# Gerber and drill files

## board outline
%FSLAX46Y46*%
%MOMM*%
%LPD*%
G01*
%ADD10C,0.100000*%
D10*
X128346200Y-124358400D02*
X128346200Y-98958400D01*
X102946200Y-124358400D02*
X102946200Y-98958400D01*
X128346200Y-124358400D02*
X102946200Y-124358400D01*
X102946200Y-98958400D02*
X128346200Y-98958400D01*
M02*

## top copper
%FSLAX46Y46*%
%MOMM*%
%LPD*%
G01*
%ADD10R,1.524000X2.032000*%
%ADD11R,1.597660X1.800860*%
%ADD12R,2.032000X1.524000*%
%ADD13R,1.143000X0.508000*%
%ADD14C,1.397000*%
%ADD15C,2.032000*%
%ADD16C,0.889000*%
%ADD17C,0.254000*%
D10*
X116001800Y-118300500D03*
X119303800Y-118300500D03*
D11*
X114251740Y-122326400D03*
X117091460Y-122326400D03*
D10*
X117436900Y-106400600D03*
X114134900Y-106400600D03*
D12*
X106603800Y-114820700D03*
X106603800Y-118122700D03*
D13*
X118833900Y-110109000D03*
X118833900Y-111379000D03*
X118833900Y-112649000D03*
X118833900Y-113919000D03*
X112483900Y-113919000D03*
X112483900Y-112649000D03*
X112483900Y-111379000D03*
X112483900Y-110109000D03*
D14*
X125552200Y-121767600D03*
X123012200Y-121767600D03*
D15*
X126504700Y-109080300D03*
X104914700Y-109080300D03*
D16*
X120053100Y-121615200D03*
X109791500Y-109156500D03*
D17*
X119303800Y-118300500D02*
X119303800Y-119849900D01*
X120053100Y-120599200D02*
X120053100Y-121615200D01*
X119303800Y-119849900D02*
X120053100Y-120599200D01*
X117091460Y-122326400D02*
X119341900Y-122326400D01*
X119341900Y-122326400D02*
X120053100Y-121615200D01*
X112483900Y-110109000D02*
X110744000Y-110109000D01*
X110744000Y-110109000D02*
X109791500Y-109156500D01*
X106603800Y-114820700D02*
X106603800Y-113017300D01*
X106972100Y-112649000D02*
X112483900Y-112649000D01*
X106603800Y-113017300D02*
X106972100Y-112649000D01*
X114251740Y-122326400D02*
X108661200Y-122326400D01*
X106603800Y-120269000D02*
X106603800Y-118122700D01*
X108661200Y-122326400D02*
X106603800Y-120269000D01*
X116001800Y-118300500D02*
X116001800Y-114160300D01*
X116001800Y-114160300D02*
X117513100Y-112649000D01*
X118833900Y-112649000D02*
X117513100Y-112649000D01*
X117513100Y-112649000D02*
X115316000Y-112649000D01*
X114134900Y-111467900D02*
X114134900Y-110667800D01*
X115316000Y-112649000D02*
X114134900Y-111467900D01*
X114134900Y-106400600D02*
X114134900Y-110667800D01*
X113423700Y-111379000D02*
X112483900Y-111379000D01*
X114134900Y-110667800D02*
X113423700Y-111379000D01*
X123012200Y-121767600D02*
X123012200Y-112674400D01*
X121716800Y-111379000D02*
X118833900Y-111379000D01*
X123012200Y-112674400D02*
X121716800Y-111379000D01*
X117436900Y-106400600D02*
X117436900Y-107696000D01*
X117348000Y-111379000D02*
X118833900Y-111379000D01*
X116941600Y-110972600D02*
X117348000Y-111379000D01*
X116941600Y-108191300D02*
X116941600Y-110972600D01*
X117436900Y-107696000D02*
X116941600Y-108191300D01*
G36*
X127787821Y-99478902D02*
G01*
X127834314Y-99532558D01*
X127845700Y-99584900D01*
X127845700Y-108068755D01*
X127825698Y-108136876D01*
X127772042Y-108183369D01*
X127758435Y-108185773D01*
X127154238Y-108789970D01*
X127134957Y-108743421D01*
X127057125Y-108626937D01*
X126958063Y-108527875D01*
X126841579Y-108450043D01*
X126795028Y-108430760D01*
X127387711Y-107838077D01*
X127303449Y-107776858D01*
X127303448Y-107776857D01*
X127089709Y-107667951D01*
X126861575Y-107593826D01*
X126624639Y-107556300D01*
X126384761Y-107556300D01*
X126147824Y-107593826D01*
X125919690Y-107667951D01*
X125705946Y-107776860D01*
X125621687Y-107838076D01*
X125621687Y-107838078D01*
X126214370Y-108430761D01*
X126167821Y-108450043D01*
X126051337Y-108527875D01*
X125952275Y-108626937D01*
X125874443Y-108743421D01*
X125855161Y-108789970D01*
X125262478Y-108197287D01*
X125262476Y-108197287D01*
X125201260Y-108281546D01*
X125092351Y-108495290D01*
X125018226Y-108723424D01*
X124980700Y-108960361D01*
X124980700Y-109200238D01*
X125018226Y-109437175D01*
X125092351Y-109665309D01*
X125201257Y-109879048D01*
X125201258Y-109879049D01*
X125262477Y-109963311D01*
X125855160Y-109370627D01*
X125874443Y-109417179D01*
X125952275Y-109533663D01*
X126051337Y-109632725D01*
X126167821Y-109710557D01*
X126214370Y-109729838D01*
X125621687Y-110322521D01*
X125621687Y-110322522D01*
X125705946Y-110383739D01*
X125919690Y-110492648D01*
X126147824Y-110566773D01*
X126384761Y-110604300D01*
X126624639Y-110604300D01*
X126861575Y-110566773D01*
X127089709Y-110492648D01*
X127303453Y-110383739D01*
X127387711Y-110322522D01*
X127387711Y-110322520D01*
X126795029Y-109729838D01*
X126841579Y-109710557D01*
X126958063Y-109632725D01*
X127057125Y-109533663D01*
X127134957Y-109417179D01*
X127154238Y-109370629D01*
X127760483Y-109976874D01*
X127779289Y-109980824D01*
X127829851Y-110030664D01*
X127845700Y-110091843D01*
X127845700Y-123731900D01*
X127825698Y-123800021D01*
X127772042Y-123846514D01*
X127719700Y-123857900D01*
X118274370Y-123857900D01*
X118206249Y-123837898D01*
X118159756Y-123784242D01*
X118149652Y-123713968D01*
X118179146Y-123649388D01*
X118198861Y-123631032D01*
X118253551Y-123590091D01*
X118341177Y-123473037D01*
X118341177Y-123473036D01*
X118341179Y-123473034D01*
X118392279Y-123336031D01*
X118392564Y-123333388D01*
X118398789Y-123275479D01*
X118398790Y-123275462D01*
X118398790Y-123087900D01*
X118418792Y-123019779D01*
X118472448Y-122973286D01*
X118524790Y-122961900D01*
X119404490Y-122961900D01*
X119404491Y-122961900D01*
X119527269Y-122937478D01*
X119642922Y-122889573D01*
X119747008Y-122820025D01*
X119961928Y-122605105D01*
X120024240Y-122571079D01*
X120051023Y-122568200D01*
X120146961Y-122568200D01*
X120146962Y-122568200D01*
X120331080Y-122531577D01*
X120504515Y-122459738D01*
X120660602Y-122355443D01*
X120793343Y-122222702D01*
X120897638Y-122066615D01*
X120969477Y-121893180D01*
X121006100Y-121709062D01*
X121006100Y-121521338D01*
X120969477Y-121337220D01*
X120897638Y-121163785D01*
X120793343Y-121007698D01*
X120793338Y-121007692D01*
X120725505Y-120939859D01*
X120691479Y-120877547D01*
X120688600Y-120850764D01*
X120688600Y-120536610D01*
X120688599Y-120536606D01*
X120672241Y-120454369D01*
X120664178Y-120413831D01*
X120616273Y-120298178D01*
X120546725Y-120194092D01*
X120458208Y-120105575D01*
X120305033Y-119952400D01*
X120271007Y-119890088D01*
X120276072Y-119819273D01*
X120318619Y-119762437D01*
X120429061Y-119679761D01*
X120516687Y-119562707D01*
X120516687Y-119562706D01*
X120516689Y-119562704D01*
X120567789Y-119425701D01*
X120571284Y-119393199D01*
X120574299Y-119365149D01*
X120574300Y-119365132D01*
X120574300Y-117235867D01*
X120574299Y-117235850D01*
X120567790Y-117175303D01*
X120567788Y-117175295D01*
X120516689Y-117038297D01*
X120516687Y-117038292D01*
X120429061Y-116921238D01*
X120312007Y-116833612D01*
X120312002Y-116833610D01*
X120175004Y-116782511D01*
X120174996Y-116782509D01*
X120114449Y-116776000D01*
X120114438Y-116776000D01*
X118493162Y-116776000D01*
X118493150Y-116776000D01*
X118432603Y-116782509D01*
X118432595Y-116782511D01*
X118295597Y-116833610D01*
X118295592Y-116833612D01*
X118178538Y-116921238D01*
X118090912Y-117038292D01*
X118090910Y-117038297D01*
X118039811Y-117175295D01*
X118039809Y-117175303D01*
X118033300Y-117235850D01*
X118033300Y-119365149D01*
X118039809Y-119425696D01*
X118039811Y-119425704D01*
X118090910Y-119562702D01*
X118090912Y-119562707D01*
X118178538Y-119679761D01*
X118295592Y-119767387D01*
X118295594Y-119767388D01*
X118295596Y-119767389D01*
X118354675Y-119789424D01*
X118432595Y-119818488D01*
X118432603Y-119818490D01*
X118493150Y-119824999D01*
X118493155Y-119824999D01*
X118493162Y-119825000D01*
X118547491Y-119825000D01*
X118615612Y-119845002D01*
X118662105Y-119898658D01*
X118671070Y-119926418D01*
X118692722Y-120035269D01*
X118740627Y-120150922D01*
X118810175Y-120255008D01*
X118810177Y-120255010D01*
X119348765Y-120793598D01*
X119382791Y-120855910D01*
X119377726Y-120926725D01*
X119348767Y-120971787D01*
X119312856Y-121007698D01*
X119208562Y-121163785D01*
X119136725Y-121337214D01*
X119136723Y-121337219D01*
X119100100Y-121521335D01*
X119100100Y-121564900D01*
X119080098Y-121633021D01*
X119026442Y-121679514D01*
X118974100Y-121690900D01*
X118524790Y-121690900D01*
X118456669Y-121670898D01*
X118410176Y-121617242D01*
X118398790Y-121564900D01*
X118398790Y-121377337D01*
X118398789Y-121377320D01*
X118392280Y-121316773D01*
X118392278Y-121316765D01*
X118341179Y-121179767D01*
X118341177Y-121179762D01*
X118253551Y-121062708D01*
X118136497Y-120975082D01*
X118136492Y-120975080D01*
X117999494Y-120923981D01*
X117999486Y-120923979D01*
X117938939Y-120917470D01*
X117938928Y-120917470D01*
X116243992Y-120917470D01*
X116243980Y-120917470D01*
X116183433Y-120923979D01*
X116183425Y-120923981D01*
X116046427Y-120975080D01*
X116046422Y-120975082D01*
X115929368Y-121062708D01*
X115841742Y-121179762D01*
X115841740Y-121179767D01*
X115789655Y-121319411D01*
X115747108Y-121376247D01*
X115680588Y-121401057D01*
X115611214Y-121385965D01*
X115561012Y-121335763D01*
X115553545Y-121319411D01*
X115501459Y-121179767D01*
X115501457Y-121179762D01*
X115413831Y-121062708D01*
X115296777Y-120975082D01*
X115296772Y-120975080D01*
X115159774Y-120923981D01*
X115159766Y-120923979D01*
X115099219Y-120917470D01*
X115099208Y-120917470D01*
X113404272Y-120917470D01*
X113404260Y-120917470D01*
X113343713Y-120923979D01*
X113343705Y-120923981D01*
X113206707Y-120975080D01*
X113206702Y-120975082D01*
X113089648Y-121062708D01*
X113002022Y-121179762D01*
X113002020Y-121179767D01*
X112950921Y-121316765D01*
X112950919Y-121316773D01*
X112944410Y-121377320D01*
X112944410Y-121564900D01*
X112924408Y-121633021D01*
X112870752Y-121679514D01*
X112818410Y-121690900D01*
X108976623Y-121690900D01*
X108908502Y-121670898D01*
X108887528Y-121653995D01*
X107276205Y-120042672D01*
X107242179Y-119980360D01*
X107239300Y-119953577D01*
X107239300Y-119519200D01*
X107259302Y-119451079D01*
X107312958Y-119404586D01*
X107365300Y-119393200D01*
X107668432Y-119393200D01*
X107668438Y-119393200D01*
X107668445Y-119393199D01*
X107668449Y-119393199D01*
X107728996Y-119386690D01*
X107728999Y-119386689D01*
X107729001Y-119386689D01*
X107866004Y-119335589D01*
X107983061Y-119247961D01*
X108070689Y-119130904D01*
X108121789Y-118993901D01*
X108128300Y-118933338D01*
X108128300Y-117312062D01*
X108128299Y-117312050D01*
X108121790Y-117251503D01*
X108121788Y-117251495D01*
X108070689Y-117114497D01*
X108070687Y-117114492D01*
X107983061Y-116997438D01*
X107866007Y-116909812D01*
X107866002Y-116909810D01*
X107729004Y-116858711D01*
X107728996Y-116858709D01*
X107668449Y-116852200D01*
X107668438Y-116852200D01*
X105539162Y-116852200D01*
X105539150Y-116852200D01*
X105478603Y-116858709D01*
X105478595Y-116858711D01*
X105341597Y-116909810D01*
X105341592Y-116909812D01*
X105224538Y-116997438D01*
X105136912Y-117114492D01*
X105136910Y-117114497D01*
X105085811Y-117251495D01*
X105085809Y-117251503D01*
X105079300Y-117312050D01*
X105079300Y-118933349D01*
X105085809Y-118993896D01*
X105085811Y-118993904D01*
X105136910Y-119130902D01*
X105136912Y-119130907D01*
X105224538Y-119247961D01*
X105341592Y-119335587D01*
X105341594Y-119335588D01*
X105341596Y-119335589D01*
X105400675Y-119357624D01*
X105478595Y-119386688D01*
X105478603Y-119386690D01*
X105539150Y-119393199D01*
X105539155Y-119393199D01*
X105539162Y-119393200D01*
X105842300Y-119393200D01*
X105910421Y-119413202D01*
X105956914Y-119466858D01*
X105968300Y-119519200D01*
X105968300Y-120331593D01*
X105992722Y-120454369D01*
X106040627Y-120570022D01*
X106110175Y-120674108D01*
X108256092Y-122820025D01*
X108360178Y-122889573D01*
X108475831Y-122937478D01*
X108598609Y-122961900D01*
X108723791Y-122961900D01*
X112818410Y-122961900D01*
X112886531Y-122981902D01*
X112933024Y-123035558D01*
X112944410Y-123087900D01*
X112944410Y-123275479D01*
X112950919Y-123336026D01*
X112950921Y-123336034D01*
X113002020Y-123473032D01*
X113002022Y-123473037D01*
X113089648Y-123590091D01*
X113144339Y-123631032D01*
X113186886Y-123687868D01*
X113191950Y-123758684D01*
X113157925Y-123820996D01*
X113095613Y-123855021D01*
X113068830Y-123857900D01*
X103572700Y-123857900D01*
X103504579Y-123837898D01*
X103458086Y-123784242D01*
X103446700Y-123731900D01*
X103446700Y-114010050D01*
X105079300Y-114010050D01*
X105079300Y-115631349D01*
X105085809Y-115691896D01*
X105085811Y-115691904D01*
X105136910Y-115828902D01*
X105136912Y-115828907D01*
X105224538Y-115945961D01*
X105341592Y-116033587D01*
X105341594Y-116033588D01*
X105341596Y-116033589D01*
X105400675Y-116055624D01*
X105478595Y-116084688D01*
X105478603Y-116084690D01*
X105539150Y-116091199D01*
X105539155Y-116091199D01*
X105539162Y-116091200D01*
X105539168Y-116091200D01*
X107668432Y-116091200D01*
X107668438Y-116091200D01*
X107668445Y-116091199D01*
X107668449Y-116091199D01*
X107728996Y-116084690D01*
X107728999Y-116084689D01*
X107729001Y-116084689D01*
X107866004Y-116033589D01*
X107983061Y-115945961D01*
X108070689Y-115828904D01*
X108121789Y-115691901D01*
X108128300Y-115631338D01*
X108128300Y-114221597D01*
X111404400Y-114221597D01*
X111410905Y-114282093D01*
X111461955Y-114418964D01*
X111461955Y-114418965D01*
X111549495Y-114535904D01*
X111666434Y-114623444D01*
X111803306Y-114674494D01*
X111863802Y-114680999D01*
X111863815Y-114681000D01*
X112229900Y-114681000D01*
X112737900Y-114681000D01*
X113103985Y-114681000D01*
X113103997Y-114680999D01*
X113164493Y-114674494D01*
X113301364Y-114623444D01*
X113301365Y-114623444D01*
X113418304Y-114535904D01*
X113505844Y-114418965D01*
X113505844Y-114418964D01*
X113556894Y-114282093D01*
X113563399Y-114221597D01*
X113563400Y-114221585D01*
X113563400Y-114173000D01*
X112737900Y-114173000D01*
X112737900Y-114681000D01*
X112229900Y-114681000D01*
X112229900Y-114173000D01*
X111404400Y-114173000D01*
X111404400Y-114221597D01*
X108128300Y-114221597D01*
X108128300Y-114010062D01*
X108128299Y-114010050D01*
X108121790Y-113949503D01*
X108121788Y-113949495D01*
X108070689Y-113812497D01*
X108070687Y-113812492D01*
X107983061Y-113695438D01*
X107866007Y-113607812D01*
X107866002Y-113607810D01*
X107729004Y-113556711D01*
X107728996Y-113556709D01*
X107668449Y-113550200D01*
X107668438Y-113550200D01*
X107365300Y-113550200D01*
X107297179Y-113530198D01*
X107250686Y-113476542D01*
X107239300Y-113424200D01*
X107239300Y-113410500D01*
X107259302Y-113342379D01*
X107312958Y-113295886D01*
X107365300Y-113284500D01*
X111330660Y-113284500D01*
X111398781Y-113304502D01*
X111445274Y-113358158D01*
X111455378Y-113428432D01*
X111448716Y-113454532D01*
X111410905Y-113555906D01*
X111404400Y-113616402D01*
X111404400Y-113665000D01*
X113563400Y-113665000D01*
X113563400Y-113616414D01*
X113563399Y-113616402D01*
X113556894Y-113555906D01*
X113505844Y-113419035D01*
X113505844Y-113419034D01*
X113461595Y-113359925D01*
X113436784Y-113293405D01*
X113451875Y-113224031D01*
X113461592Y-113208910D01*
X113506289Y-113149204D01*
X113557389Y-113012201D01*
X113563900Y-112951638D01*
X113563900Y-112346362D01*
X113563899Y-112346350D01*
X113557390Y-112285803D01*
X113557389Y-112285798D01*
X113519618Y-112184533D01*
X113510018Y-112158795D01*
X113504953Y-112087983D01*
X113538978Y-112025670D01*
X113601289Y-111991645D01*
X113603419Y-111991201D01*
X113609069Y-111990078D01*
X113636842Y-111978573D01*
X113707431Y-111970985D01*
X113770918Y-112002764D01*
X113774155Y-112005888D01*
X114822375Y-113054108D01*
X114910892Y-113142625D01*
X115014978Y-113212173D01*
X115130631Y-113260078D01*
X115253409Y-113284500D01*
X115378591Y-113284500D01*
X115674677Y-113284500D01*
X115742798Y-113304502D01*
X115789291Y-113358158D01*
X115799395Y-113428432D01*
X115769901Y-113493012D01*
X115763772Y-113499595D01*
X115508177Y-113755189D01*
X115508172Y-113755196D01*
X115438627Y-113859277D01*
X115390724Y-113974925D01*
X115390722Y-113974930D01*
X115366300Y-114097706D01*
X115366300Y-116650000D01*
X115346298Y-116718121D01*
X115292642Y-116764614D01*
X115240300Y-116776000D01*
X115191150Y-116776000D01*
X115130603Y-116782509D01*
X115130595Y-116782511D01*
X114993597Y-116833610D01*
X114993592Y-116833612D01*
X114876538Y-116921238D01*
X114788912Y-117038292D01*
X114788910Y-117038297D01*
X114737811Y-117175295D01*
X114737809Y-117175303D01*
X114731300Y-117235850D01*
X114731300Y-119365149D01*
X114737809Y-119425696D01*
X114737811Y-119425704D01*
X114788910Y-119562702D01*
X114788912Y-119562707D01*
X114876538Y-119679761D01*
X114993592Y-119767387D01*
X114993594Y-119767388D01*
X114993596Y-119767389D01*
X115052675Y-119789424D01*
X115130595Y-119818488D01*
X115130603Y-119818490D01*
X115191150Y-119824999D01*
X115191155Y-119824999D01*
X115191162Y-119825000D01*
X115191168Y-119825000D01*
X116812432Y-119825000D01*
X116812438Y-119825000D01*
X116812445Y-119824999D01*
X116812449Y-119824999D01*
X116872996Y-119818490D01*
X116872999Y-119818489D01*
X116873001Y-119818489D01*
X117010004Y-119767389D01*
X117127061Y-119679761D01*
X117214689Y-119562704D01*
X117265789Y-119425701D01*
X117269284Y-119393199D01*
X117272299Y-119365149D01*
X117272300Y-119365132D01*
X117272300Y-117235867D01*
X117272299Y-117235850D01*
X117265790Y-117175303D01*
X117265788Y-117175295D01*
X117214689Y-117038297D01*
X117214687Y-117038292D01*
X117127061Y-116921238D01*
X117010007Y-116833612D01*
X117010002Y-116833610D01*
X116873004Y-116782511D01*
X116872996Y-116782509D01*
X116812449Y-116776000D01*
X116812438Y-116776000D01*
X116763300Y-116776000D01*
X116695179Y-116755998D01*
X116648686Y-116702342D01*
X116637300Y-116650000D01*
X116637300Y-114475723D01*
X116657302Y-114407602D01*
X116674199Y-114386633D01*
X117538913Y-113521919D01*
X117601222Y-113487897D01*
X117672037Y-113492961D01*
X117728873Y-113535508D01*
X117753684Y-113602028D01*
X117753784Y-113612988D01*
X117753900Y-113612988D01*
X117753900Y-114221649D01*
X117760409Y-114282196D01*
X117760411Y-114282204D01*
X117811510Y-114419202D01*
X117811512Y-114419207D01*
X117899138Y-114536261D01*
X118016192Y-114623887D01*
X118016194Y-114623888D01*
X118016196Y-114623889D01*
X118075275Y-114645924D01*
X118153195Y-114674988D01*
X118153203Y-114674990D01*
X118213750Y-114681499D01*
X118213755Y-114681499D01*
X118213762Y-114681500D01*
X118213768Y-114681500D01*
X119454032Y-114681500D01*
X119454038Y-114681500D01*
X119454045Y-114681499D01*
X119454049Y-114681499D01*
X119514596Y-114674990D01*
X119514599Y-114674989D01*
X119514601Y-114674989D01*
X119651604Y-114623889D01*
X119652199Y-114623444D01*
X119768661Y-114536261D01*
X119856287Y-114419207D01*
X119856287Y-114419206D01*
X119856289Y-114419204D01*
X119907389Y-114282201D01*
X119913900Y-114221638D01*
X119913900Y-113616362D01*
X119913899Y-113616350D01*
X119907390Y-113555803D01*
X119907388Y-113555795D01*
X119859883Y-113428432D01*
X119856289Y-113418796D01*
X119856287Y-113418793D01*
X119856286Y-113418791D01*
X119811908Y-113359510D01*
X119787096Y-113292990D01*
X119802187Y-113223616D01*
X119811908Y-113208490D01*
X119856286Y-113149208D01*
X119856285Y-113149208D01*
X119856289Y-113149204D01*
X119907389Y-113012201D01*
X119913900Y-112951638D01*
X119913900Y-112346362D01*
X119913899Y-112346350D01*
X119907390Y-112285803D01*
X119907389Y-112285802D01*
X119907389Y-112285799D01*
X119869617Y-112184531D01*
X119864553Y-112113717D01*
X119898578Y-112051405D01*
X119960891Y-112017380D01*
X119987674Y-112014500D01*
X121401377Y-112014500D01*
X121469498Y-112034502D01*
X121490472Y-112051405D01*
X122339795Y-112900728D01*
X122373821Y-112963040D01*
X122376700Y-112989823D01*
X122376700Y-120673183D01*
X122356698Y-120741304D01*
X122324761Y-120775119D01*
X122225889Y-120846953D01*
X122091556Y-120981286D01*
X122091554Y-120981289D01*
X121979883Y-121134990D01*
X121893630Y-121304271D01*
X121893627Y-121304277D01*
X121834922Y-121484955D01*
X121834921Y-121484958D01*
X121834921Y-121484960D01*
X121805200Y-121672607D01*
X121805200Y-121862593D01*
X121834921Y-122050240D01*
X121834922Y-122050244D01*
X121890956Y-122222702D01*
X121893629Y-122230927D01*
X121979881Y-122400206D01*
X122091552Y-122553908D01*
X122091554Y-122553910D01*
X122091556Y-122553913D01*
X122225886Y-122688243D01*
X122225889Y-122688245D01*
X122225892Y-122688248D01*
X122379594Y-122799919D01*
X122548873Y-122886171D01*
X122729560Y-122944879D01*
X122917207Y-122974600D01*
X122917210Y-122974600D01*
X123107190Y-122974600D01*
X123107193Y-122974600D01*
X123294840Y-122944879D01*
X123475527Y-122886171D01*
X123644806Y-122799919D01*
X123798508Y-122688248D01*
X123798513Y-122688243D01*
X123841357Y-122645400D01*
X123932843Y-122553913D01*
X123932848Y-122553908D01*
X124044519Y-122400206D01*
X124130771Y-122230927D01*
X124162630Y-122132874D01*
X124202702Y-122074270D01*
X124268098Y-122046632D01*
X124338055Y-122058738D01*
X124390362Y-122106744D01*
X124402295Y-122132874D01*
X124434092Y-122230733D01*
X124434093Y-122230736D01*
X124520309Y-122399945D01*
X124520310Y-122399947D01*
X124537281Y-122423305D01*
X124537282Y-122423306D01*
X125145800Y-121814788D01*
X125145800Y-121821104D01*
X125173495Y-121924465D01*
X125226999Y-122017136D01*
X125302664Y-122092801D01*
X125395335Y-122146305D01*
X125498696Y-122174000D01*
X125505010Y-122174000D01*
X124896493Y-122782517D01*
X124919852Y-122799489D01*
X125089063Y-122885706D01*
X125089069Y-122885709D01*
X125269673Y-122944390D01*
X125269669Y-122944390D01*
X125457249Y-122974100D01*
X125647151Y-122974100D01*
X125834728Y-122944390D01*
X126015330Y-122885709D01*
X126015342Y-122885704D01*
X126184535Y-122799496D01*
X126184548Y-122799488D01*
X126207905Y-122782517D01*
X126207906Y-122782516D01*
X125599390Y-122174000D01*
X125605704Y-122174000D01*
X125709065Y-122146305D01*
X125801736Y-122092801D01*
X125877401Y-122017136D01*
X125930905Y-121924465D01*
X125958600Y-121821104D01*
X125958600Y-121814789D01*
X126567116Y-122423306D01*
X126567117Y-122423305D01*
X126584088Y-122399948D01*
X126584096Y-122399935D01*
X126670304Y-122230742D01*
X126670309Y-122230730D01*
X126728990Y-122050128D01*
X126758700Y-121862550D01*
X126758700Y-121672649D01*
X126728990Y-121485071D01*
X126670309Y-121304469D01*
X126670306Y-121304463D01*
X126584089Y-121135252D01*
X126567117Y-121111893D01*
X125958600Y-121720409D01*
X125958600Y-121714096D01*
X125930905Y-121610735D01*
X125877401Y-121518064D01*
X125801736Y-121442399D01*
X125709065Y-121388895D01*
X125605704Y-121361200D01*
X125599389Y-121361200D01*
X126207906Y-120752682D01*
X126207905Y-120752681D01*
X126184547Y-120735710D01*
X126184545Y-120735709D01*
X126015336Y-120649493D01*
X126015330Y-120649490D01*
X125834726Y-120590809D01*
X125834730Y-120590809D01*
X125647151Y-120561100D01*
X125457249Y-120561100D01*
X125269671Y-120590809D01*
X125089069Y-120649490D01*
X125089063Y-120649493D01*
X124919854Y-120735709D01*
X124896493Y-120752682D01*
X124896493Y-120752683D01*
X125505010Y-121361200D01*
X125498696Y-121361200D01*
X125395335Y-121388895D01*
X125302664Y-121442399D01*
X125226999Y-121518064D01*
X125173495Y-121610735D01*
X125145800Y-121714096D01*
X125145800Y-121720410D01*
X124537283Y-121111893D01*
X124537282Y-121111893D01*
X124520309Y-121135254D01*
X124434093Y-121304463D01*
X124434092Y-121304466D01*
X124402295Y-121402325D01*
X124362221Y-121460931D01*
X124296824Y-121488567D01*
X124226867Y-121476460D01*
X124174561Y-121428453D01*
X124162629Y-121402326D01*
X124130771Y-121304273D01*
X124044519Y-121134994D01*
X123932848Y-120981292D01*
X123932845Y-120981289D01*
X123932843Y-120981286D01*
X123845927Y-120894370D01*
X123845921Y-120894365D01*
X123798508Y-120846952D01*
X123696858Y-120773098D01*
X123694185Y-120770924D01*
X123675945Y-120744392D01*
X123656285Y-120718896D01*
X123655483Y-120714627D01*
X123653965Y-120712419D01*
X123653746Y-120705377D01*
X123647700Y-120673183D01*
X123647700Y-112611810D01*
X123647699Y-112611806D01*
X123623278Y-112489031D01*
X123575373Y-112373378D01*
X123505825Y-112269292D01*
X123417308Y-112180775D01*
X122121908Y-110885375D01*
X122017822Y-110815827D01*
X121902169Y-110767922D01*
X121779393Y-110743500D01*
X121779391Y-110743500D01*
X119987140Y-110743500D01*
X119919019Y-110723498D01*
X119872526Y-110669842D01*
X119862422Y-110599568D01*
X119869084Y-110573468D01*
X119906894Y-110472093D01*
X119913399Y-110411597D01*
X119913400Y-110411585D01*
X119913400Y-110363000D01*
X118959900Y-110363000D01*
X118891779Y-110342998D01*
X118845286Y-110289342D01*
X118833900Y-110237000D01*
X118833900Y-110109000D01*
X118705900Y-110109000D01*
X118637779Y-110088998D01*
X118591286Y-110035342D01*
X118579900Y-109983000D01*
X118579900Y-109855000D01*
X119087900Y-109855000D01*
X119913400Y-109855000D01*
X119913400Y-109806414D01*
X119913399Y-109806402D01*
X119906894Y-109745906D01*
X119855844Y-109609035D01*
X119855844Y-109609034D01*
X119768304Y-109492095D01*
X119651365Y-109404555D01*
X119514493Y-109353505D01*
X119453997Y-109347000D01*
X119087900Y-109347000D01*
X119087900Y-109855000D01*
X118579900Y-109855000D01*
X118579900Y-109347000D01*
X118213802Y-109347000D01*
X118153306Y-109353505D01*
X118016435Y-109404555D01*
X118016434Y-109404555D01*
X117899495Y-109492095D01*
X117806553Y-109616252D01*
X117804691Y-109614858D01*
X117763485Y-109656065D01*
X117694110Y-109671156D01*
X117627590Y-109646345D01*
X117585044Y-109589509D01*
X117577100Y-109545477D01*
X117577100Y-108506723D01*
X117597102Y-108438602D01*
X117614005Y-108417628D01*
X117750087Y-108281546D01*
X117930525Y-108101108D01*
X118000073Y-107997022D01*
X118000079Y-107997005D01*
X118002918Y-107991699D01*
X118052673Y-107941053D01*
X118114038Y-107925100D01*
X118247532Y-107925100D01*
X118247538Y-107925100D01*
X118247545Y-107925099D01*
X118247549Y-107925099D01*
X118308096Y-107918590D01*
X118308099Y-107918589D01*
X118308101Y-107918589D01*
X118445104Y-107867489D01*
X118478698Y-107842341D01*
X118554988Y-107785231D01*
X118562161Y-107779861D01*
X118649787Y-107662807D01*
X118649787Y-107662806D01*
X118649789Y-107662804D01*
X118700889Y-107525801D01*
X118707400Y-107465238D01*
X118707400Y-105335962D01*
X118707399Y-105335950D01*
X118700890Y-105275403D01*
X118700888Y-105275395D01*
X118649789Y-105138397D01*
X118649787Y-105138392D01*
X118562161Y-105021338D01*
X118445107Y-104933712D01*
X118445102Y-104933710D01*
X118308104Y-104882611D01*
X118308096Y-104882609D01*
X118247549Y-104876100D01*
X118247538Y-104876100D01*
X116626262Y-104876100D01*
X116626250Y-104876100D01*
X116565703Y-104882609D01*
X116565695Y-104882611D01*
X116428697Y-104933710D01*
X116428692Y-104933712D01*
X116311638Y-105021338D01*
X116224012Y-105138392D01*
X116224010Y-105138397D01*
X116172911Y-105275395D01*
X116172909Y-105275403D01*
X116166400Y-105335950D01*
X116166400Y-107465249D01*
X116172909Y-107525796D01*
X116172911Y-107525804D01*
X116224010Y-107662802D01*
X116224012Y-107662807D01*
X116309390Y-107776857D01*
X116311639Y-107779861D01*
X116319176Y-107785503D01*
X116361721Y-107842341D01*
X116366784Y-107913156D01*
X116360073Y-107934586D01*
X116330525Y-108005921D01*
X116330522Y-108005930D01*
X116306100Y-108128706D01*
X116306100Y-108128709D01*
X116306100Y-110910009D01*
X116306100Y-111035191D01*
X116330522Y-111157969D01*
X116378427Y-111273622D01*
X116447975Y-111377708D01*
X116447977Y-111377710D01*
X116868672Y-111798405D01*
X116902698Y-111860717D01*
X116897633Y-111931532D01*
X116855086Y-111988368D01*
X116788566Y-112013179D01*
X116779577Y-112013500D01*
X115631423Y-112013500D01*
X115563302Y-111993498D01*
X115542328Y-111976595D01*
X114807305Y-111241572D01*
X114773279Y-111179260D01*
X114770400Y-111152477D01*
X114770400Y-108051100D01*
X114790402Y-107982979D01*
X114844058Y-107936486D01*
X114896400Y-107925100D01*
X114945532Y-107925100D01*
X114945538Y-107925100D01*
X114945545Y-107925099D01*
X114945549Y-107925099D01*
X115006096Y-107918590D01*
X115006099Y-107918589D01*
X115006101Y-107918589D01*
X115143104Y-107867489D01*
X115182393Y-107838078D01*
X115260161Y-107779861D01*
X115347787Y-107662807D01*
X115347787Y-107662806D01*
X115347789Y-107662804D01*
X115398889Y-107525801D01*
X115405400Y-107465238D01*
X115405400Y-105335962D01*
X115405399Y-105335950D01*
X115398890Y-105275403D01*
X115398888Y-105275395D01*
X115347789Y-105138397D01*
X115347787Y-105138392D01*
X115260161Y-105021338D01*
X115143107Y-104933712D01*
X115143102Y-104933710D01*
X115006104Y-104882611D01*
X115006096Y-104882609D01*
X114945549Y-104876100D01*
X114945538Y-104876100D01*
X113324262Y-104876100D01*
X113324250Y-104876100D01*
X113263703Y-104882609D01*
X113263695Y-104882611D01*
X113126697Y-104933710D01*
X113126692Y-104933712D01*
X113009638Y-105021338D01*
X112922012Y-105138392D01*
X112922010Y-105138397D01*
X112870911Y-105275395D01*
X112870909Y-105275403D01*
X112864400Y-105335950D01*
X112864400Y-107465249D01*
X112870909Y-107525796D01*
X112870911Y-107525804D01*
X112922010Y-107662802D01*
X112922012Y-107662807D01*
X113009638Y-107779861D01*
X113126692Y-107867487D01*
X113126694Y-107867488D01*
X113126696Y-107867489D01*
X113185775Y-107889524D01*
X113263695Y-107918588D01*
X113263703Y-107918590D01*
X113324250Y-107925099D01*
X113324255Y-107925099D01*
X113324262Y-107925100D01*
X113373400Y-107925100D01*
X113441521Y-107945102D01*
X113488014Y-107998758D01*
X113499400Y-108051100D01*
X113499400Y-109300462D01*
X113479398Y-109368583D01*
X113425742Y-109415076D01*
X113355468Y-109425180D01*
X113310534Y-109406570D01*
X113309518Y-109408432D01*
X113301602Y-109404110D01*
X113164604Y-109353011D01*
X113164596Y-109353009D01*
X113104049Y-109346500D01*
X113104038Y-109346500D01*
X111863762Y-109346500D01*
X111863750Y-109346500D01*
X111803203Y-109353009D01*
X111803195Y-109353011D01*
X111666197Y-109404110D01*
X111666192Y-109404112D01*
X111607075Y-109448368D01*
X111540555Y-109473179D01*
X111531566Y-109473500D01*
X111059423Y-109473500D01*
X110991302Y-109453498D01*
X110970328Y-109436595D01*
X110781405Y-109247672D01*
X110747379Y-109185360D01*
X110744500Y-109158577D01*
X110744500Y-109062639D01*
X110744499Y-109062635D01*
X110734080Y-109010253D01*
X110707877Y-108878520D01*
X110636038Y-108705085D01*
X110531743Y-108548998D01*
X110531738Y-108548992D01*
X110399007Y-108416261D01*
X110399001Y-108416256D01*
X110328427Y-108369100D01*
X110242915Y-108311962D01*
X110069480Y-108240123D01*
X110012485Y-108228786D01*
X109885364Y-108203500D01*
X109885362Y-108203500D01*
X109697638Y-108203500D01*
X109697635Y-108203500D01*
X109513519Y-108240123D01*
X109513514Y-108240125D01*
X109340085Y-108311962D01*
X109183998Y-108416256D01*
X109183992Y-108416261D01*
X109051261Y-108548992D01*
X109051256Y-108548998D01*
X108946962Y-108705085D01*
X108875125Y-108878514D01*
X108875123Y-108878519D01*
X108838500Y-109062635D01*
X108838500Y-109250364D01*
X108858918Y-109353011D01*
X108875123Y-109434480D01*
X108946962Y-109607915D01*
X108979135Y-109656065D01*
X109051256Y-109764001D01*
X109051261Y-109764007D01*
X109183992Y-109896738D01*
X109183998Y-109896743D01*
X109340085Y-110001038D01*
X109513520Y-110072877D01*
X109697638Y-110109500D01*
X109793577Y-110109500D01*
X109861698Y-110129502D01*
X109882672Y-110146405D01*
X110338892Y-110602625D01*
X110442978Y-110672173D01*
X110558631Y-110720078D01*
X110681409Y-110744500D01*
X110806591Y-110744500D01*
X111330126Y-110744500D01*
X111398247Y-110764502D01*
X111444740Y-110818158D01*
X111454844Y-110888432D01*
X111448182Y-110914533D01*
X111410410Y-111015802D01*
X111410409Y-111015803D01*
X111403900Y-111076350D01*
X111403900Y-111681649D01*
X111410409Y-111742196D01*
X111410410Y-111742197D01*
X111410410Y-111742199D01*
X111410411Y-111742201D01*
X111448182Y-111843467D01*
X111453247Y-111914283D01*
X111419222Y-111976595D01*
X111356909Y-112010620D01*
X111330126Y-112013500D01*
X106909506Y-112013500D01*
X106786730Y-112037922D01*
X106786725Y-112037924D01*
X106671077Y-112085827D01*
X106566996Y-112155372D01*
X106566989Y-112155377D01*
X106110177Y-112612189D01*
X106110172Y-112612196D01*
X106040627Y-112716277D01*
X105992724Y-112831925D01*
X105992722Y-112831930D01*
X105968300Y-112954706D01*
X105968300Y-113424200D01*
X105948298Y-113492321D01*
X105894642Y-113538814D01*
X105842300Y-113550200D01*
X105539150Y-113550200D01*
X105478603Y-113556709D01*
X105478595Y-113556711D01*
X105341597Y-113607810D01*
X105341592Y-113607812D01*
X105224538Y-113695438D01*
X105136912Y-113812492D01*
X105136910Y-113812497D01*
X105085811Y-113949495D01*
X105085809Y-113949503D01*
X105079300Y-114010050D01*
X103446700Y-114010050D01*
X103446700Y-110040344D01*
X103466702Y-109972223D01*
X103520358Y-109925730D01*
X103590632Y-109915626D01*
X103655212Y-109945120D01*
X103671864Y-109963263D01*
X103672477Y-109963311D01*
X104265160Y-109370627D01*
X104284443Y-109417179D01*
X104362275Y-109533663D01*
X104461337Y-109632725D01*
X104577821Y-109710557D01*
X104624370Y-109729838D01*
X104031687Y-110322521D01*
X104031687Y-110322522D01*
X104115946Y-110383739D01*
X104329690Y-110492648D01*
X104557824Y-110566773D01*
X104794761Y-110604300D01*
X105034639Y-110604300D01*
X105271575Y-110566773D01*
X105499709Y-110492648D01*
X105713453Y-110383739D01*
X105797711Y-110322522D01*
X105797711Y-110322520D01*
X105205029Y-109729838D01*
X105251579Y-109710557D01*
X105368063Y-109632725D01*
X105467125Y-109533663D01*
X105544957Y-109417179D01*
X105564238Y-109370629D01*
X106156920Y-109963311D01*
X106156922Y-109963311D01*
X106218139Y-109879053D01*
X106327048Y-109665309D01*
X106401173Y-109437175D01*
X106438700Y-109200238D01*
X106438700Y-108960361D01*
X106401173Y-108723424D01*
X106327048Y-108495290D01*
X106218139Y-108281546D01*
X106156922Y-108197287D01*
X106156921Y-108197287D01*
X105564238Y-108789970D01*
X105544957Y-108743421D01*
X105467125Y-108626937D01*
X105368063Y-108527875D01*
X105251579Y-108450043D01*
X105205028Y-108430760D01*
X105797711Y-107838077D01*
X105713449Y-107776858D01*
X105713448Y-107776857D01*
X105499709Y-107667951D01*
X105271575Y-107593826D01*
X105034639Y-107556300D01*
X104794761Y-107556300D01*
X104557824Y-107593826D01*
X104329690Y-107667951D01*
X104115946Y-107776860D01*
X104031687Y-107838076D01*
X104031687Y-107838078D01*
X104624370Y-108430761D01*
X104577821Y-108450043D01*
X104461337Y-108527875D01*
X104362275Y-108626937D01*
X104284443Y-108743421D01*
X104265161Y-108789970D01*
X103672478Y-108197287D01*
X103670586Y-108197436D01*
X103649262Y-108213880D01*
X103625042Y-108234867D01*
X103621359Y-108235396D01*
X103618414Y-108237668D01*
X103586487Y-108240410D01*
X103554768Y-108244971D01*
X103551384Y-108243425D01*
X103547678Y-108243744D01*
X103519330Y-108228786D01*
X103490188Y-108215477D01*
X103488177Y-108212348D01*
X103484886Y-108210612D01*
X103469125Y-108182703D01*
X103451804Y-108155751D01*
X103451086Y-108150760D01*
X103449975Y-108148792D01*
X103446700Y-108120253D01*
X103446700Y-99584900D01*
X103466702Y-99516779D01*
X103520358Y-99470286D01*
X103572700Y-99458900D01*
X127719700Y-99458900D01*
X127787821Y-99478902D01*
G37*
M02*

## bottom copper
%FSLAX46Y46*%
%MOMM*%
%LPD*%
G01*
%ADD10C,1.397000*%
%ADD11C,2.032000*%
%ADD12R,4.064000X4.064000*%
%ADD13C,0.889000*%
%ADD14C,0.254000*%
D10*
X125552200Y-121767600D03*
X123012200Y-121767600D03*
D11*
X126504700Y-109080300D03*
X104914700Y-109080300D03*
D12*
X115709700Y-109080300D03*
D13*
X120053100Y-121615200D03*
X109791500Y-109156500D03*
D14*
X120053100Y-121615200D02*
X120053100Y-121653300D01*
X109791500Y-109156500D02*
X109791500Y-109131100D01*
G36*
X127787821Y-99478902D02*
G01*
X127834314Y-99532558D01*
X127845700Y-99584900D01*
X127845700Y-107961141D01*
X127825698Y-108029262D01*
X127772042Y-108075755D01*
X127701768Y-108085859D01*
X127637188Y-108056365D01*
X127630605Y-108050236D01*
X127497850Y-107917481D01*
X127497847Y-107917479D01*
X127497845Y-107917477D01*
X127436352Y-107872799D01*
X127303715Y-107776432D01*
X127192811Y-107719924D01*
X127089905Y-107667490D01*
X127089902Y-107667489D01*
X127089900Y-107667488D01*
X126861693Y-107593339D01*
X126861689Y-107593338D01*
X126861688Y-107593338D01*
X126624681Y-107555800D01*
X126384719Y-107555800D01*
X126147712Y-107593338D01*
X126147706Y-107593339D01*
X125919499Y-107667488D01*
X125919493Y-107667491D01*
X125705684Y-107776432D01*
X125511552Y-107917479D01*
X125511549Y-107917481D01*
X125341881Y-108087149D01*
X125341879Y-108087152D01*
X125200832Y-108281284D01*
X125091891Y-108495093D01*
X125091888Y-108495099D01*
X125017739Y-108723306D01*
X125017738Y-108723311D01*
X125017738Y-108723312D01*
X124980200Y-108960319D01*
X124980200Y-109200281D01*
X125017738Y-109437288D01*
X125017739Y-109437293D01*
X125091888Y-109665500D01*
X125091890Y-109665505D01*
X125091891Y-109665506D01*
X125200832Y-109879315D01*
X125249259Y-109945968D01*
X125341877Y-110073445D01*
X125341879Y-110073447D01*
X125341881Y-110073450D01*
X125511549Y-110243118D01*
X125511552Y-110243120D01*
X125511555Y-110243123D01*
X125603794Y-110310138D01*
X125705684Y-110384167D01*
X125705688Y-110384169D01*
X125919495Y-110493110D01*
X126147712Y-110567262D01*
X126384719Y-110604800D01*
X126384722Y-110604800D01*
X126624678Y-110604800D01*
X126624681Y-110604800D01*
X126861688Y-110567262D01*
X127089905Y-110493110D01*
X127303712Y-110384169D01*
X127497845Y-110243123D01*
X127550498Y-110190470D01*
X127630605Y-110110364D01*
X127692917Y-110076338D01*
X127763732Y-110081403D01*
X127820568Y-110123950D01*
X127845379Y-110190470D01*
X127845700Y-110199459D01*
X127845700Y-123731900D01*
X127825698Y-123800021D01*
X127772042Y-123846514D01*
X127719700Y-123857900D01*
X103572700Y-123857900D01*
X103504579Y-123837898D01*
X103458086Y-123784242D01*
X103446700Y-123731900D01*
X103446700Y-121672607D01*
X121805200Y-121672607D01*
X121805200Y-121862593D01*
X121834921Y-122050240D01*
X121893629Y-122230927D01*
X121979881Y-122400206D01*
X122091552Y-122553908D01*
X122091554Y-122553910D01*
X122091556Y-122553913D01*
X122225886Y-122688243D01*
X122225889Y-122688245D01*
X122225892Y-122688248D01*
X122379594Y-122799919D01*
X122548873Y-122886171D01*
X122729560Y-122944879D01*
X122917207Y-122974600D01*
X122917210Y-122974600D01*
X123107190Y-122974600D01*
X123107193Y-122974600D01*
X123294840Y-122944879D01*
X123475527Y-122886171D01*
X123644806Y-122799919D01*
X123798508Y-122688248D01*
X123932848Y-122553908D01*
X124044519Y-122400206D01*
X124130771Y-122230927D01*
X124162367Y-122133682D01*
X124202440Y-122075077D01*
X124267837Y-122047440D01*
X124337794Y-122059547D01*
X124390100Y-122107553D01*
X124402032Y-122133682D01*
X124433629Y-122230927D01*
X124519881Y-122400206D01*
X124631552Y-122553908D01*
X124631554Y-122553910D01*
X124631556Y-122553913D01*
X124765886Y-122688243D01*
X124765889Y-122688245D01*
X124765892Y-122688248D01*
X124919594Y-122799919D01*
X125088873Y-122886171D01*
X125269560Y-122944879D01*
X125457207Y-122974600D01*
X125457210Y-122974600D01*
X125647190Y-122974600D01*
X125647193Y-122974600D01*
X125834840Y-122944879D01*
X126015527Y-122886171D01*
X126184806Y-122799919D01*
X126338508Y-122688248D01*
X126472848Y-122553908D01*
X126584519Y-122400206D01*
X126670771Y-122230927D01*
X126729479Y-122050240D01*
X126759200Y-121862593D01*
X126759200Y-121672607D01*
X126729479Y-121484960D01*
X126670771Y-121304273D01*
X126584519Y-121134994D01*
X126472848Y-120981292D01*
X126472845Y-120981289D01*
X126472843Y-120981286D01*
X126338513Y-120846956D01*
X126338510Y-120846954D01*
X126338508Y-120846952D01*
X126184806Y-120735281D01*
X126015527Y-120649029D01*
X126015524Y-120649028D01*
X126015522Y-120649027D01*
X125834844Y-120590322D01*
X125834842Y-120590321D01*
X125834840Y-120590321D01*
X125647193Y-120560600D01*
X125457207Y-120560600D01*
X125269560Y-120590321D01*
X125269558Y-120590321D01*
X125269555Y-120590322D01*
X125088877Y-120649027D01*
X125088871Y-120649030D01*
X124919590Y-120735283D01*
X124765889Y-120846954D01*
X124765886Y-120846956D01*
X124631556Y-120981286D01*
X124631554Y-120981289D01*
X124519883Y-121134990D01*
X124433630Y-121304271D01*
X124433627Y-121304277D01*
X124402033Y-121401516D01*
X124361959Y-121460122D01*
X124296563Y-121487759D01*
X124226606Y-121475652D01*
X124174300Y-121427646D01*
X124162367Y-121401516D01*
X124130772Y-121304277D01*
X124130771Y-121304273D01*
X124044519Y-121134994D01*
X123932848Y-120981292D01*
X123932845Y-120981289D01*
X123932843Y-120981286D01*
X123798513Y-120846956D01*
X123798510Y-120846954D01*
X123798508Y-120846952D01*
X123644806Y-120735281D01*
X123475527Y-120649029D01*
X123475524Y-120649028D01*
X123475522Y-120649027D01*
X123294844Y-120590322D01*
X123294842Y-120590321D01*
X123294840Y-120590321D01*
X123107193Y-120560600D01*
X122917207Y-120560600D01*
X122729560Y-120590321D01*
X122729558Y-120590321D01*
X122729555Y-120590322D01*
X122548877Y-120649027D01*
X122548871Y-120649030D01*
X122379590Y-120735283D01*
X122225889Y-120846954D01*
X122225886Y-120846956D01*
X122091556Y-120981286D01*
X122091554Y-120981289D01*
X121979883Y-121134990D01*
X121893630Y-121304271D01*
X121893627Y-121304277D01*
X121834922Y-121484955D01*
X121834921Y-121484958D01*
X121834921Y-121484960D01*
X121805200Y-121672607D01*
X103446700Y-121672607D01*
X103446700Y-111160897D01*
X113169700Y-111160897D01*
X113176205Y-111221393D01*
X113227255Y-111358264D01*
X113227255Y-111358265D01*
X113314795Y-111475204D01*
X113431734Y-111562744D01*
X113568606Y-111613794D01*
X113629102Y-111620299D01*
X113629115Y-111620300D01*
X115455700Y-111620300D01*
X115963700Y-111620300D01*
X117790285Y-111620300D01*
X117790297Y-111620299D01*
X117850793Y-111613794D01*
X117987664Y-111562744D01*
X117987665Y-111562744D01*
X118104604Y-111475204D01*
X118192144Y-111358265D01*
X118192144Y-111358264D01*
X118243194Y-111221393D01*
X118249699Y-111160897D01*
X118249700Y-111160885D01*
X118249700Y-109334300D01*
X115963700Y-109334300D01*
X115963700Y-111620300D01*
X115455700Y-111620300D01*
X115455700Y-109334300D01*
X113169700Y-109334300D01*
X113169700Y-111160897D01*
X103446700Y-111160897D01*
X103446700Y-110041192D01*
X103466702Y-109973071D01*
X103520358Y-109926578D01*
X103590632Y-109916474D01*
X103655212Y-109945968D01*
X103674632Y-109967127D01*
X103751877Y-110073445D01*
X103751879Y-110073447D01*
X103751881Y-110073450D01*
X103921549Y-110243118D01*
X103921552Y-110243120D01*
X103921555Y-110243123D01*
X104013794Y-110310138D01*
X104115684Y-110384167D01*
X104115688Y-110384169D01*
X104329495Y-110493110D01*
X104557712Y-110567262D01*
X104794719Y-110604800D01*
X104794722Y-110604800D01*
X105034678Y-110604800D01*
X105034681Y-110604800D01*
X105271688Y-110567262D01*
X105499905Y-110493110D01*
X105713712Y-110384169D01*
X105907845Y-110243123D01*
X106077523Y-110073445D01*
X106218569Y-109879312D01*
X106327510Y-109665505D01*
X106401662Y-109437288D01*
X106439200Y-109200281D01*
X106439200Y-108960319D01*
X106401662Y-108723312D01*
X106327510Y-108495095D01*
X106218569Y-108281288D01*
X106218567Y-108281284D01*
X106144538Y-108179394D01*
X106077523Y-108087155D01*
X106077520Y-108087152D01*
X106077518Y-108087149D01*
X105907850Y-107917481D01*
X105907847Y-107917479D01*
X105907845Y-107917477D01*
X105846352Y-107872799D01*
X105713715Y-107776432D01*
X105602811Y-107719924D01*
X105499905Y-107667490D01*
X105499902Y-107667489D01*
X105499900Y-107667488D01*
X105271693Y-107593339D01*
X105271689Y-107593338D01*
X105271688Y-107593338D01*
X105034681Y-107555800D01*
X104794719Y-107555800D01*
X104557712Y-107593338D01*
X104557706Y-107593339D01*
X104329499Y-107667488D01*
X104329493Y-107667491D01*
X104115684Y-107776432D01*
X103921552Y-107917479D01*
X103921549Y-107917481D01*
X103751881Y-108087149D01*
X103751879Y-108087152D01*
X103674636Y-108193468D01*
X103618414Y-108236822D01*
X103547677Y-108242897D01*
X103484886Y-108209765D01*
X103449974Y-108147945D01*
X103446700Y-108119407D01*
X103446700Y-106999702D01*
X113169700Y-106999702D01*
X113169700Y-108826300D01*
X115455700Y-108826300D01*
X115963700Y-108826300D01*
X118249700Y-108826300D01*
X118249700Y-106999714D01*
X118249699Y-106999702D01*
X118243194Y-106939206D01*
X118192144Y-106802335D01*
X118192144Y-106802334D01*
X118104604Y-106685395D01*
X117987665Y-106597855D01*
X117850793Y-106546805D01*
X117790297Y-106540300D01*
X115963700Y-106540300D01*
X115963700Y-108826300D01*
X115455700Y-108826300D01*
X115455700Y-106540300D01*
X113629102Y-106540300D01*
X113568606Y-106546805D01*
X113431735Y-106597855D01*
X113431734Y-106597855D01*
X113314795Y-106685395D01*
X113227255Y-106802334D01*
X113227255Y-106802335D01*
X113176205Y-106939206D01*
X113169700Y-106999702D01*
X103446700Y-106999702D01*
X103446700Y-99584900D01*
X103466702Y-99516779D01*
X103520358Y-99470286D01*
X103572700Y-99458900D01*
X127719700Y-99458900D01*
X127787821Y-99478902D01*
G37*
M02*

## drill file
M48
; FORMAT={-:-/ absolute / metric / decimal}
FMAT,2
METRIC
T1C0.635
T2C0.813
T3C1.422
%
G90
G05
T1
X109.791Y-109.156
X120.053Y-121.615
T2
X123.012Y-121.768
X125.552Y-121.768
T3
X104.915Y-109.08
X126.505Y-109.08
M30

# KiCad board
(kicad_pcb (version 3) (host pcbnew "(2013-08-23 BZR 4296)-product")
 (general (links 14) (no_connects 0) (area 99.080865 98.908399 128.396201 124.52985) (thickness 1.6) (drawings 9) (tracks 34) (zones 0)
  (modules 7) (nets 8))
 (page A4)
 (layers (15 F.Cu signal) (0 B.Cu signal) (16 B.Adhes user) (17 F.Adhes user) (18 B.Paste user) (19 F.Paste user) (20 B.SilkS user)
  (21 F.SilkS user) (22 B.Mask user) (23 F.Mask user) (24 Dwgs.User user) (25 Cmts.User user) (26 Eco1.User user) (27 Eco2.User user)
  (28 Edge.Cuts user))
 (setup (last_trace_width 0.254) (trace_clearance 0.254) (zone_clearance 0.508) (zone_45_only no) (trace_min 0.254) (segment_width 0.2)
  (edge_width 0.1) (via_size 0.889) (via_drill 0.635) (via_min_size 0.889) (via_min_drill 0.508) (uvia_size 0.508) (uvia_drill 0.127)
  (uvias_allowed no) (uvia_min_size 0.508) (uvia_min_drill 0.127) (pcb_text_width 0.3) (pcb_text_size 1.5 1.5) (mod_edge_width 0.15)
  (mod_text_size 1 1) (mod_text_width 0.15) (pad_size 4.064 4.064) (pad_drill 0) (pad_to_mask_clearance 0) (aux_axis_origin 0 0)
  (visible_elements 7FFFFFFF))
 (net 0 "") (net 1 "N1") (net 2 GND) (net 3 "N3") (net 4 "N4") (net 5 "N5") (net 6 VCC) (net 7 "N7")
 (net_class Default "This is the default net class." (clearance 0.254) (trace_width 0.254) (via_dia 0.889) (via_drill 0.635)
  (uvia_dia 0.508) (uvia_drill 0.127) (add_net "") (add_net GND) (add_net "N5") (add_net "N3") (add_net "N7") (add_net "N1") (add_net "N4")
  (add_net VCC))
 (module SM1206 (layer F.Cu) (at 117.6528 118.3005)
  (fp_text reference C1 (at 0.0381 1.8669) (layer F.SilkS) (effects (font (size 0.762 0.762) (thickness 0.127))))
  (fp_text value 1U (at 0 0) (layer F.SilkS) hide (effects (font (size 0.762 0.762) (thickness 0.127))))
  (pad 1 smd rect (at -1.651 0) (size 1.524 2.032) (layers F.Cu F.Paste F.Mask) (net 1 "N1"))
  (pad 2 smd rect (at 1.651 0) (size 1.524 2.032) (layers F.Cu F.Paste F.Mask) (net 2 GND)))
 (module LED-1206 (layer F.Cu) (at 115.6716 122.3264)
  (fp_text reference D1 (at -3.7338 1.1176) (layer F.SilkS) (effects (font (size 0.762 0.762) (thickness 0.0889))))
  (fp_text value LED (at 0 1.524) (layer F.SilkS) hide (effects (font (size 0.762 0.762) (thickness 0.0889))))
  (pad 1 smd rect (at -1.41986 0) (size 1.59766 1.80086) (layers F.Cu F.Paste F.Mask) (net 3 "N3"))
  (pad 2 smd rect (at 1.41986 0) (size 1.59766 1.80086) (layers F.Cu F.Paste F.Mask) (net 2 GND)))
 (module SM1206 (layer F.Cu) (at 115.7859 106.4006 180)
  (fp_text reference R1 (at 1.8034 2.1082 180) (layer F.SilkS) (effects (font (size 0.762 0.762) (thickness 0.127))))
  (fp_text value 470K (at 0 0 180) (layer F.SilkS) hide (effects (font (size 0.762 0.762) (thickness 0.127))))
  (pad 1 smd rect (at -1.651 0 180) (size 1.524 2.032) (layers F.Cu F.Paste F.Mask) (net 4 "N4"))
  (pad 2 smd rect (at 1.651 0 180) (size 1.524 2.032) (layers F.Cu F.Paste F.Mask) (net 1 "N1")))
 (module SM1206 (layer F.Cu) (at 106.6038 116.4717 270)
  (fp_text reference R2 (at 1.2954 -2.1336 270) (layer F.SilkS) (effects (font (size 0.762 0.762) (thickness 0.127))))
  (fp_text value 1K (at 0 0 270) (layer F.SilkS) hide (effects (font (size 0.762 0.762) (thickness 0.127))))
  (pad 1 smd rect (at -1.651 0 270) (size 1.524 2.032) (layers F.Cu F.Paste F.Mask) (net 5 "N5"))
  (pad 2 smd rect (at 1.651 0 270) (size 1.524 2.032) (layers F.Cu F.Paste F.Mask) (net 3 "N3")))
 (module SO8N (layer F.Cu) (at 115.6589 112.014 270)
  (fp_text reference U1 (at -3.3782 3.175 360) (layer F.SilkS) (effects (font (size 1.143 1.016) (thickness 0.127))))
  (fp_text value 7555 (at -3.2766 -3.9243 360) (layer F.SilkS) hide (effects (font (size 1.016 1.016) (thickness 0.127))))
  (pad 8 smd rect (at -1.905 -3.175 270) (size 0.508 1.143) (layers F.Cu F.Paste F.Mask) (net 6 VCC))
  (pad 7 smd rect (at -0.635 -3.175 270) (size 0.508 1.143) (layers F.Cu F.Paste F.Mask) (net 4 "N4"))
  (pad 6 smd rect (at 0.635 -3.175 270) (size 0.508 1.143) (layers F.Cu F.Paste F.Mask) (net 1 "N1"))
  (pad 5 smd rect (at 1.905 -3.175 270) (size 0.508 1.143) (layers F.Cu F.Paste F.Mask) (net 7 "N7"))
  (pad 4 smd rect (at 1.905 3.175 270) (size 0.508 1.143) (layers F.Cu F.Paste F.Mask) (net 6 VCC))
  (pad 3 smd rect (at 0.635 3.175 270) (size 0.508 1.143) (layers F.Cu F.Paste F.Mask) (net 5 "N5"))
  (pad 2 smd rect (at -0.635 3.175 270) (size 0.508 1.143) (layers F.Cu F.Paste F.Mask) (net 1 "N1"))
  (pad 1 smd rect (at -1.905 3.175 270) (size 0.508 1.143) (layers F.Cu F.Paste F.Mask) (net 2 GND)))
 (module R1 (layer F.Cu) (at 124.2822 121.7676 180) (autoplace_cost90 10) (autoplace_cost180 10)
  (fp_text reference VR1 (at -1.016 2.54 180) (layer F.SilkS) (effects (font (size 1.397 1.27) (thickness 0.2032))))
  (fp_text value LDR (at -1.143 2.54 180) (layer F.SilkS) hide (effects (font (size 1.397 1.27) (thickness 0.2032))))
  (pad 1 thru_hole circle (at -1.27 0 180) (size 1.397 1.397) (drill 0.8128) (layers *.Cu *.Mask F.SilkS) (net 6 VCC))
  (pad 2 thru_hole circle (at 1.27 0 180) (size 1.397 1.397) (drill 0.8128) (layers *.Cu *.Mask F.SilkS) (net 4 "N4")))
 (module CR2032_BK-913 (layer B.Cu) (at 115.7097 109.0803 180)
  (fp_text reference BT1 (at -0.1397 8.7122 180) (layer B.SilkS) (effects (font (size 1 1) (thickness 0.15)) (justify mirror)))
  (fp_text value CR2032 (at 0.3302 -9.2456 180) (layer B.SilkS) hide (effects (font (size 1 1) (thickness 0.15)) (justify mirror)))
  (pad 1 thru_hole circle (at -10.795 0 180) (size 2.032 2.032) (drill 1.4224) (layers *.Cu *.Mask B.SilkS) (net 6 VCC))
  (pad 1 thru_hole circle (at 10.795 0 180) (size 2.032 2.032) (drill 1.4224) (layers *.Cu *.Mask B.SilkS) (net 6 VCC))
  (pad 2 smd rect (at 0 0 180) (size 4.064 4.064) (layers B.Cu B.Paste B.Mask) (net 2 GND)))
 (gr_line (start 128.3462 124.3584) (end 128.3462 98.9584) (angle 90) (layer Edge.Cuts) (width 0.1))
 (gr_line (start 102.9462 124.3584) (end 102.9462 98.9584) (angle 90) (layer Edge.Cuts) (width 0.1))
 (gr_line (start 128.3462 124.3584) (end 102.9462 124.3584) (angle 90) (layer Edge.Cuts) (width 0.1))
 (gr_line (start 102.9462 98.9584) (end 128.3462 98.9584) (angle 90) (layer Edge.Cuts) (width 0.1))
 (segment (start 119.3038 118.3005) (end 119.3038 119.8499) (width 0.254) (layer F.Cu) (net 2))
 (segment (start 120.0531 120.5992) (end 120.0531 121.6152) (width 0.254) (layer F.Cu) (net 2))
 (segment (start 119.3038 119.8499) (end 120.0531 120.5992) (width 0.254) (layer F.Cu) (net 2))
 (segment (start 117.09146 122.3264) (end 119.3419 122.3264) (width 0.254) (layer F.Cu) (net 2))
 (segment (start 120.0531 121.6152) (end 120.0531 121.6533) (width 0.254) (layer B.Cu) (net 2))
 (via (at 120.0531 121.6152) (size 0.889) (layers F.Cu B.Cu) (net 2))
 (segment (start 119.3419 122.3264) (end 120.0531 121.6152) (width 0.254) (layer F.Cu) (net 2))
 (segment (start 112.4839 110.109) (end 110.744 110.109) (width 0.254) (layer F.Cu) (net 2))
 (segment (start 109.7915 109.1565) (end 109.7915 109.1311) (width 0.254) (layer B.Cu) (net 2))
 (via (at 109.7915 109.1565) (size 0.889) (layers F.Cu B.Cu) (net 2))
 (segment (start 110.744 110.109) (end 109.7915 109.1565) (width 0.254) (layer F.Cu) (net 2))
 (segment (start 106.6038 114.8207) (end 106.6038 113.0173) (width 0.254) (layer F.Cu) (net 5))
 (segment (start 106.9721 112.649) (end 112.4839 112.649) (width 0.254) (layer F.Cu) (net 5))
 (segment (start 106.6038 113.0173) (end 106.9721 112.649) (width 0.254) (layer F.Cu) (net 5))
 (segment (start 114.25174 122.3264) (end 108.6612 122.3264) (width 0.254) (layer F.Cu) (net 3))
 (segment (start 106.6038 120.269) (end 106.6038 118.1227) (width 0.254) (layer F.Cu) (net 3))
 (segment (start 108.6612 122.3264) (end 106.6038 120.269) (width 0.254) (layer F.Cu) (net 3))
 (segment (start 116.0018 118.3005) (end 116.0018 114.1603) (width 0.254) (layer F.Cu) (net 1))
 (segment (start 116.0018 114.1603) (end 117.5131 112.649) (width 0.254) (layer F.Cu) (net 1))
 (segment (start 118.8339 112.649) (end 117.5131 112.649) (width 0.254) (layer F.Cu) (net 1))
 (segment (start 117.5131 112.649) (end 115.316 112.649) (width 0.254) (layer F.Cu) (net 1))
 (segment (start 114.1349 111.4679) (end 114.1349 110.6678) (width 0.254) (layer F.Cu) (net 1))
 (segment (start 115.316 112.649) (end 114.1349 111.4679) (width 0.254) (layer F.Cu) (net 1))
 (segment (start 114.1349 106.4006) (end 114.1349 110.6678) (width 0.254) (layer F.Cu) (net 1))
 (segment (start 113.4237 111.379) (end 112.4839 111.379) (width 0.254) (layer F.Cu) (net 1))
 (segment (start 114.1349 110.6678) (end 113.4237 111.379) (width 0.254) (layer F.Cu) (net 1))
 (segment (start 123.0122 121.7676) (end 123.0122 112.6744) (width 0.254) (layer F.Cu) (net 4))
 (segment (start 121.7168 111.379) (end 118.8339 111.379) (width 0.254) (layer F.Cu) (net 4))
 (segment (start 123.0122 112.6744) (end 121.7168 111.379) (width 0.254) (layer F.Cu) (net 4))
 (segment (start 117.4369 106.4006) (end 117.4369 107.696) (width 0.254) (layer F.Cu) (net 4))
 (segment (start 117.348 111.379) (end 118.8339 111.379) (width 0.254) (layer F.Cu) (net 4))
 (segment (start 116.9416 110.9726) (end 117.348 111.379) (width 0.254) (layer F.Cu) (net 4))
 (segment (start 116.9416 108.1913) (end 116.9416 110.9726) (width 0.254) (layer F.Cu) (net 4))
 (segment (start 117.4369 107.696) (end 116.9416 108.1913) (width 0.254) (layer F.Cu) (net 4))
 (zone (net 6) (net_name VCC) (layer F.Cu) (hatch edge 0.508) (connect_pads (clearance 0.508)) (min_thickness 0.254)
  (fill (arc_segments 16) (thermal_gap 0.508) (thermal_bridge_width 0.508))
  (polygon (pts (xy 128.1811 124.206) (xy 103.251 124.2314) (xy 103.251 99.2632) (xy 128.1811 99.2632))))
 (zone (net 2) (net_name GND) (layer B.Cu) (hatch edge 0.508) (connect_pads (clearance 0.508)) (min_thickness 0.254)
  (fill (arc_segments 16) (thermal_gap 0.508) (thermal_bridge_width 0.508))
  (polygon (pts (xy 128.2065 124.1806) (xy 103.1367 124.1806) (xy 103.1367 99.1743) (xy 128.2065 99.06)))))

